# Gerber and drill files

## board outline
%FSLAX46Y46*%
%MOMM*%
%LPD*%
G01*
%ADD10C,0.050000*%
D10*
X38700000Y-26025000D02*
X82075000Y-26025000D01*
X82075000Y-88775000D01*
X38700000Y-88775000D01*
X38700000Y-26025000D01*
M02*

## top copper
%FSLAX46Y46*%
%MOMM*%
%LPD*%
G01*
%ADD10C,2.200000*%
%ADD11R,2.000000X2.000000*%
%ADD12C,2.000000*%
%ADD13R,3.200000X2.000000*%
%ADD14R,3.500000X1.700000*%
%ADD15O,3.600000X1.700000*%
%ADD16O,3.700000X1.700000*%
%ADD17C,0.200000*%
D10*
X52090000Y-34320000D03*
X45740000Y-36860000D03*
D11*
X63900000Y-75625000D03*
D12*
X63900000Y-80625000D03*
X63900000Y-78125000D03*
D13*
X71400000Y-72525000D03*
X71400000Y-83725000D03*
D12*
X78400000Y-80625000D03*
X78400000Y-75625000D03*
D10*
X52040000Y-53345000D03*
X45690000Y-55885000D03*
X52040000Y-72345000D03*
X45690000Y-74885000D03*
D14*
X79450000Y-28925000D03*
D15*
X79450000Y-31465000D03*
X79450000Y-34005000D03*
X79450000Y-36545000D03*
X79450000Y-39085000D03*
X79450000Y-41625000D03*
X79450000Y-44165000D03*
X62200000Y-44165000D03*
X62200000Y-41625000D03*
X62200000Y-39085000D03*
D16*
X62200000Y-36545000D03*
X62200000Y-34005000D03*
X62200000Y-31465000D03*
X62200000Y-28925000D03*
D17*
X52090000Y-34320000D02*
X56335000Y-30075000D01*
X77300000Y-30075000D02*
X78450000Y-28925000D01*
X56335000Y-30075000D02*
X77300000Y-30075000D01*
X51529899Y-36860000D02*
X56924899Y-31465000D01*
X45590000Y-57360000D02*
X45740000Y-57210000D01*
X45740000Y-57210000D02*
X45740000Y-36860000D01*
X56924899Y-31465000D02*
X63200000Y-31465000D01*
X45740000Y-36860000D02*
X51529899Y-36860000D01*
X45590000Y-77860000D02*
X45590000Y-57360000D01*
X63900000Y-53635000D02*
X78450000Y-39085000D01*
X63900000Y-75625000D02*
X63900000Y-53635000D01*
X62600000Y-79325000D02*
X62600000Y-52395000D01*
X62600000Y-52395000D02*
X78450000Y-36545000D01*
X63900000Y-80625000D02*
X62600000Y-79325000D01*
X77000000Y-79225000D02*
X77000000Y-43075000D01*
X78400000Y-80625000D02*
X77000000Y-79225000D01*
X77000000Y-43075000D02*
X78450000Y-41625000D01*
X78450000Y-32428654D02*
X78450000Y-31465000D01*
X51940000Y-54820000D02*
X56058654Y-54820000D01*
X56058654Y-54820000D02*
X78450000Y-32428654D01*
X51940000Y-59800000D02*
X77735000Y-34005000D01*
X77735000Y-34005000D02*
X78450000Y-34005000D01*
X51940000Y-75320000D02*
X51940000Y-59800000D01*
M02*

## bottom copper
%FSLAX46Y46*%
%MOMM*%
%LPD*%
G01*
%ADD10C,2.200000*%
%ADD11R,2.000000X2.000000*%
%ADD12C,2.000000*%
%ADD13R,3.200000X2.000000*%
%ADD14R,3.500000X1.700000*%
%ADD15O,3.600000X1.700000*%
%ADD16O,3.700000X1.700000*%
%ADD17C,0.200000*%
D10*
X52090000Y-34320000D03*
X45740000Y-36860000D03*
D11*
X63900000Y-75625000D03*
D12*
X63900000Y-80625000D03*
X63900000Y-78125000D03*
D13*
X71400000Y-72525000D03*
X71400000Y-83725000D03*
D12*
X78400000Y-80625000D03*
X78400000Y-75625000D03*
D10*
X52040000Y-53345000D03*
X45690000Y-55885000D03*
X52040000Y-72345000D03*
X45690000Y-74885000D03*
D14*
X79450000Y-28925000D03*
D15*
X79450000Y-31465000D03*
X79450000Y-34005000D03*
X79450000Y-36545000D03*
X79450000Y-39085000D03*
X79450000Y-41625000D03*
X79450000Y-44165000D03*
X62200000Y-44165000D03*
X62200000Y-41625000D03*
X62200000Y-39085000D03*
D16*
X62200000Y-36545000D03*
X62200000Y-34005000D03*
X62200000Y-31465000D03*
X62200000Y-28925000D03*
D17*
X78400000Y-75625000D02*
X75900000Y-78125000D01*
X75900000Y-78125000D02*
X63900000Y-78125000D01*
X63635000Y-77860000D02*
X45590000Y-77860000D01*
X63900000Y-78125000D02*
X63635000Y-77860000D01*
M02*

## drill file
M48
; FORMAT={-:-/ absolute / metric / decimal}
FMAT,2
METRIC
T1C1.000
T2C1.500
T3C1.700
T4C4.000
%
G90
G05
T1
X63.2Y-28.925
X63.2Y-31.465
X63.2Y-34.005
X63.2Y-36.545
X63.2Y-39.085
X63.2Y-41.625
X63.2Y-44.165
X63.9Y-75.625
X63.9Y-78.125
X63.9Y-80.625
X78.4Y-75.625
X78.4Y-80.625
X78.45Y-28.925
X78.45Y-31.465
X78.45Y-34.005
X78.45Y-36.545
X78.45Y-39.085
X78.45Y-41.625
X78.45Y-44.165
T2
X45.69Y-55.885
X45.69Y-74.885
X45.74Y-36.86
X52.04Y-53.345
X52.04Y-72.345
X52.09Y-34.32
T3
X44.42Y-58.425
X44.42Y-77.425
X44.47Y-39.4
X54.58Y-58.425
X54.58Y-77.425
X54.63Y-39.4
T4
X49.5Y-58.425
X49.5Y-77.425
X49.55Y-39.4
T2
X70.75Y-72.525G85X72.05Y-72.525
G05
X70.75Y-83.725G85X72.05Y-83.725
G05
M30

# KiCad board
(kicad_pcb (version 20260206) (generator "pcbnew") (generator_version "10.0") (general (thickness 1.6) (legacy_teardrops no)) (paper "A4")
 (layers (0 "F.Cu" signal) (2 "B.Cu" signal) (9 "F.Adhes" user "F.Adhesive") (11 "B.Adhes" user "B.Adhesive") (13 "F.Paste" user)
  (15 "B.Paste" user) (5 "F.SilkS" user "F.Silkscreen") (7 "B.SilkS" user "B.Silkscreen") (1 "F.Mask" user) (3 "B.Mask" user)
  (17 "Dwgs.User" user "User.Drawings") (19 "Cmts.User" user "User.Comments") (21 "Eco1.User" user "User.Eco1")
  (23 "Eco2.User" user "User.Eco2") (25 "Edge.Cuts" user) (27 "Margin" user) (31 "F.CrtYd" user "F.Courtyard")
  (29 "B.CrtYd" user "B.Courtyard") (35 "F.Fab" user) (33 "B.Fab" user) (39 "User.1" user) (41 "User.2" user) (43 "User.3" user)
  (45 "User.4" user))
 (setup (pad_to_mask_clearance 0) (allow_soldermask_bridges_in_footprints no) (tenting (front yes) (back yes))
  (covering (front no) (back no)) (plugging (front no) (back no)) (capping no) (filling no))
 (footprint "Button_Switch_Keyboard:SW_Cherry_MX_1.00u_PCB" (layer "F.Cu") (at 52.09 34.32)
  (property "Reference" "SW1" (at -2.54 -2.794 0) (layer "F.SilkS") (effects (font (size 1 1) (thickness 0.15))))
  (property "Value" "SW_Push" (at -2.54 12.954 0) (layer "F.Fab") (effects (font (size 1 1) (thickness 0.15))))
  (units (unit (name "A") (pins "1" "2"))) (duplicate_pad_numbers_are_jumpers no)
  (pad "" np_thru_hole circle (at -7.62 5.08) (size 1.7 1.7) (drill 1.7) (layers "*.Cu" "*.Mask"))
  (pad "" np_thru_hole circle (at -2.54 5.08) (size 4 4) (drill 4) (layers "*.Cu" "*.Mask"))
  (pad "" np_thru_hole circle (at 2.54 5.08) (size 1.7 1.7) (drill 1.7) (layers "*.Cu" "*.Mask"))
  (pad "1" thru_hole circle (at 0 0) (size 2.2 2.2) (drill 1.5) (layers "*.Cu" "*.Mask") (remove_unused_layers no)
   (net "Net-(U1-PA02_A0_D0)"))
  (pad "2" thru_hole circle (at -6.35 2.54) (size 2.2 2.2) (drill 1.5) (layers "*.Cu" "*.Mask") (remove_unused_layers no) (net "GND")))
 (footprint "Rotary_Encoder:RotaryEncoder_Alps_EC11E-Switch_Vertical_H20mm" (layer "F.Cu") (at 63.9 75.625)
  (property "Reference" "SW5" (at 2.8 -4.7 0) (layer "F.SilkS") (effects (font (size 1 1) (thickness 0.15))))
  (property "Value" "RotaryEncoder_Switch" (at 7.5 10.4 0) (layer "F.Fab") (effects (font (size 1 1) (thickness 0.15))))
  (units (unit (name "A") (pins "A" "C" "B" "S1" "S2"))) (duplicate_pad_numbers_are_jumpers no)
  (pad "A" thru_hole rect (at 0 0) (size 2 2) (drill 1) (layers "*.Cu" "*.Mask") (remove_unused_layers no) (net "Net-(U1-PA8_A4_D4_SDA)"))
  (pad "B" thru_hole circle (at 0 5) (size 2 2) (drill 1) (layers "*.Cu" "*.Mask") (remove_unused_layers no) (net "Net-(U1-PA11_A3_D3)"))
  (pad "C" thru_hole circle (at 0 2.5) (size 2 2) (drill 1) (layers "*.Cu" "*.Mask") (remove_unused_layers no) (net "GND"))
  (pad "MP" thru_hole rect (at 7.5 -3.1) (size 3.2 2) (drill oval 2.8 1.5) (layers "*.Cu" "*.Mask") (remove_unused_layers no))
  (pad "MP" thru_hole rect (at 7.5 8.1) (size 3.2 2) (drill oval 2.8 1.5) (layers "*.Cu" "*.Mask") (remove_unused_layers no))
  (pad "S1" thru_hole circle (at 14.5 5) (size 2 2) (drill 1) (layers "*.Cu" "*.Mask") (remove_unused_layers no)
   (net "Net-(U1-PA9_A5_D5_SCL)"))
  (pad "S2" thru_hole circle (at 14.5 0) (size 2 2) (drill 1) (layers "*.Cu" "*.Mask") (remove_unused_layers no) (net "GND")))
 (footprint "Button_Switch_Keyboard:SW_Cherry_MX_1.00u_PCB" (layer "F.Cu") (at 52.04 53.345)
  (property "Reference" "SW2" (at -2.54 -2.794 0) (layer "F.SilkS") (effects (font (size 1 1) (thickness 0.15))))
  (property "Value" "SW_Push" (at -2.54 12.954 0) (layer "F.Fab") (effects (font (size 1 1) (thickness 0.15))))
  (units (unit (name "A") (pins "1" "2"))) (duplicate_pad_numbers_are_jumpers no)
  (pad "" np_thru_hole circle (at -7.62 5.08) (size 1.7 1.7) (drill 1.7) (layers "*.Cu" "*.Mask"))
  (pad "" np_thru_hole circle (at -2.54 5.08) (size 4 4) (drill 4) (layers "*.Cu" "*.Mask"))
  (pad "" np_thru_hole circle (at 2.54 5.08) (size 1.7 1.7) (drill 1.7) (layers "*.Cu" "*.Mask"))
  (pad "1" thru_hole circle (at 0 0) (size 2.2 2.2) (drill 1.5) (layers "*.Cu" "*.Mask") (remove_unused_layers no)
   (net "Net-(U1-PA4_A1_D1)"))
  (pad "2" thru_hole circle (at -6.35 2.54) (size 2.2 2.2) (drill 1.5) (layers "*.Cu" "*.Mask") (remove_unused_layers no) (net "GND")))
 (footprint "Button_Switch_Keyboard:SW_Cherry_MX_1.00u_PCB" (layer "F.Cu") (at 52.04 72.345)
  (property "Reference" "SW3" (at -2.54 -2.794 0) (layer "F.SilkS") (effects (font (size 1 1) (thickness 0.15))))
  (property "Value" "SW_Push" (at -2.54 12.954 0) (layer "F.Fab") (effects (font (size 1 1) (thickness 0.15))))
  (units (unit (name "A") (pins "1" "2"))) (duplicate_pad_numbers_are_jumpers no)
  (pad "" np_thru_hole circle (at -7.62 5.08) (size 1.7 1.7) (drill 1.7) (layers "*.Cu" "*.Mask"))
  (pad "" np_thru_hole circle (at -2.54 5.08) (size 4 4) (drill 4) (layers "*.Cu" "*.Mask"))
  (pad "" np_thru_hole circle (at 2.54 5.08) (size 1.7 1.7) (drill 1.7) (layers "*.Cu" "*.Mask"))
  (pad "1" thru_hole circle (at 0 0) (size 2.2 2.2) (drill 1.5) (layers "*.Cu" "*.Mask") (remove_unused_layers no)
   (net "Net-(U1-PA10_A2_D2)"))
  (pad "2" thru_hole circle (at -6.35 2.54) (size 2.2 2.2) (drill 1.5) (layers "*.Cu" "*.Mask") (remove_unused_layers no) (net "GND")))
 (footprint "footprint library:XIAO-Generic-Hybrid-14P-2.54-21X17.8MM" (layer "B.Cu") (at 70.825 36.545 180)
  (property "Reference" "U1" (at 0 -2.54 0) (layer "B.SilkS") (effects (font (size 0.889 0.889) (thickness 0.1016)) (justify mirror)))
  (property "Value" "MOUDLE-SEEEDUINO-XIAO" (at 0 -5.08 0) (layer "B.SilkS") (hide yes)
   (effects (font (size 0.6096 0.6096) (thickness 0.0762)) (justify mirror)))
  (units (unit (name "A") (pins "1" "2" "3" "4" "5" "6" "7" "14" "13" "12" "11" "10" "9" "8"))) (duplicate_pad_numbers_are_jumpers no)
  (pad "1" thru_hole rect (at -7.625 7.62 180) (size 3.5 1.7) (drill 1 (offset -1 0)) (layers "*.Cu" "*.Mask") (remove_unused_layers no)
   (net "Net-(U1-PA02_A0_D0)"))
  (pad "2" thru_hole oval (at -7.625 5.08 180) (size 3.6 1.7) (drill 1 (offset -1 0)) (layers "*.Cu" "*.Mask") (remove_unused_layers no)
   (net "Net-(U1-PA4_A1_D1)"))
  (pad "3" thru_hole oval (at -7.625 2.54 180) (size 3.6 1.7) (drill 1 (offset -1 0)) (layers "*.Cu" "*.Mask") (remove_unused_layers no)
   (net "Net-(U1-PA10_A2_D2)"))
  (pad "4" thru_hole oval (at -7.625 0 180) (size 3.6 1.7) (drill 1 (offset -1 0)) (layers "*.Cu" "*.Mask") (remove_unused_layers no)
   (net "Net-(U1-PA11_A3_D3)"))
  (pad "5" thru_hole oval (at -7.625 -2.54 180) (size 3.6 1.7) (drill 1 (offset -1 0)) (layers "*.Cu" "*.Mask") (remove_unused_layers no)
   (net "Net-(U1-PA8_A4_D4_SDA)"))
  (pad "6" thru_hole oval (at -7.625 -5.08) (size 3.6 1.7) (drill 1 (offset 1 0)) (layers "*.Cu" "*.Mask") (remove_unused_layers no)
   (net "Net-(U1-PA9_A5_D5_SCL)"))
  (pad "7" thru_hole oval (at -7.625 -7.62 180) (size 3.6 1.7) (drill 1 (offset -1 0)) (layers "*.Cu" "*.Mask") (remove_unused_layers no)
   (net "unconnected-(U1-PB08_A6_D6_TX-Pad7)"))
  (pad "8" thru_hole oval (at 7.625 -7.62 180) (size 3.6 1.7) (drill 1 (offset 1 0)) (layers "*.Cu" "*.Mask") (remove_unused_layers no)
   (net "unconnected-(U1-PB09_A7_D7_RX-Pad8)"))
  (pad "9" thru_hole oval (at 7.625 -5.08 180) (size 3.6 1.7) (drill 1 (offset 1 0)) (layers "*.Cu" "*.Mask") (remove_unused_layers no)
   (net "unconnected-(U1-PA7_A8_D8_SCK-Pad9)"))
  (pad "10" thru_hole oval (at 7.625 -2.54 180) (size 3.6 1.7) (drill 1 (offset 1 0)) (layers "*.Cu" "*.Mask") (remove_unused_layers no)
   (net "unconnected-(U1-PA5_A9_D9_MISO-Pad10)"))
  (pad "11" thru_hole oval (at 7.625 0 180) (size 3.7 1.7) (drill 1 (offset 1 0)) (layers "*.Cu" "*.Mask") (remove_unused_layers no)
   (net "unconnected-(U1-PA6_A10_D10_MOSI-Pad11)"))
  (pad "12" thru_hole oval (at 7.625 2.54 180) (size 3.7 1.7) (drill 1 (offset 1 0)) (layers "*.Cu" "*.Mask") (remove_unused_layers no)
   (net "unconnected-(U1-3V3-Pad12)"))
  (pad "13" thru_hole oval (at 7.625 5.08 180) (size 3.7 1.7) (drill 1 (offset 1 0)) (layers "*.Cu" "*.Mask") (remove_unused_layers no)
   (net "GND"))
  (pad "14" thru_hole oval (at 7.625 7.62 180) (size 3.7 1.7) (drill 1 (offset 1 0)) (layers "*.Cu" "*.Mask") (remove_unused_layers no)
   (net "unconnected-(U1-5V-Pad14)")))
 (gr_rect (start 38.7 26.025) (end 82.075 88.775) (stroke (width 0.05) (type default)) (fill no) (layer "Edge.Cuts"))
 (segment (start 52.09 34.32) (end 56.335 30.075) (width 0.2) (layer "F.Cu") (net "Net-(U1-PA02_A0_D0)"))
 (segment (start 77.3 30.075) (end 78.45 28.925) (width 0.2) (layer "F.Cu") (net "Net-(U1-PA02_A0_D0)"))
 (segment (start 56.335 30.075) (end 77.3 30.075) (width 0.2) (layer "F.Cu") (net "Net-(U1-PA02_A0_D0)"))
 (segment (start 51.529899 36.86) (end 56.924899 31.465) (width 0.2) (layer "F.Cu") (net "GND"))
 (segment (start 45.59 57.36) (end 45.74 57.21) (width 0.2) (layer "F.Cu") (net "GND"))
 (segment (start 45.74 57.21) (end 45.74 36.86) (width 0.2) (layer "F.Cu") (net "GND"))
 (segment (start 56.924899 31.465) (end 63.2 31.465) (width 0.2) (layer "F.Cu") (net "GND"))
 (segment (start 45.74 36.86) (end 51.529899 36.86) (width 0.2) (layer "F.Cu") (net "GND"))
 (segment (start 45.59 77.86) (end 45.59 57.36) (width 0.2) (layer "F.Cu") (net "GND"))
 (segment (start 78.4 75.625) (end 75.9 78.125) (width 0.2) (layer "B.Cu") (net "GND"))
 (segment (start 75.9 78.125) (end 63.9 78.125) (width 0.2) (layer "B.Cu") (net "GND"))
 (segment (start 63.635 77.86) (end 45.59 77.86) (width 0.2) (layer "B.Cu") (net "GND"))
 (segment (start 63.9 78.125) (end 63.635 77.86) (width 0.2) (layer "B.Cu") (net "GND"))
 (segment (start 63.9 53.635) (end 78.45 39.085) (width 0.2) (layer "F.Cu") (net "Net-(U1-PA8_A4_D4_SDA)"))
 (segment (start 63.9 75.625) (end 63.9 53.635) (width 0.2) (layer "F.Cu") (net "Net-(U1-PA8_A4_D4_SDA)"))
 (segment (start 62.6 79.325) (end 62.6 52.395) (width 0.2) (layer "F.Cu") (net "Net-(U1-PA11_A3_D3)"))
 (segment (start 62.6 52.395) (end 78.45 36.545) (width 0.2) (layer "F.Cu") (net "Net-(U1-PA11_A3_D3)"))
 (segment (start 63.9 80.625) (end 62.6 79.325) (width 0.2) (layer "F.Cu") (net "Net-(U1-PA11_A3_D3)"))
 (segment (start 77 79.225) (end 77 43.075) (width 0.2) (layer "F.Cu") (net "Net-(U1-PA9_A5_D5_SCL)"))
 (segment (start 78.4 80.625) (end 77 79.225) (width 0.2) (layer "F.Cu") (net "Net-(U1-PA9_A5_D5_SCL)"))
 (segment (start 77 43.075) (end 78.45 41.625) (width 0.2) (layer "F.Cu") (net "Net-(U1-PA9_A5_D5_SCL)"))
 (segment (start 78.45 32.428654) (end 78.45 31.465) (width 0.2) (layer "F.Cu") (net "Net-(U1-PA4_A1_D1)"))
 (segment (start 51.94 54.82) (end 56.058654 54.82) (width 0.2) (layer "F.Cu") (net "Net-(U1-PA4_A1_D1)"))
 (segment (start 56.058654 54.82) (end 78.45 32.428654) (width 0.2) (layer "F.Cu") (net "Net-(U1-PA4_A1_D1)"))
 (segment (start 51.94 59.8) (end 77.735 34.005) (width 0.2) (layer "F.Cu") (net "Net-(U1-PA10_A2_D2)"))
 (segment (start 77.735 34.005) (end 78.45 34.005) (width 0.2) (layer "F.Cu") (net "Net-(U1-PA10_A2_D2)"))
 (segment (start 51.94 75.32) (end 51.94 59.8) (width 0.2) (layer "F.Cu") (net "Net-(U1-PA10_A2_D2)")))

